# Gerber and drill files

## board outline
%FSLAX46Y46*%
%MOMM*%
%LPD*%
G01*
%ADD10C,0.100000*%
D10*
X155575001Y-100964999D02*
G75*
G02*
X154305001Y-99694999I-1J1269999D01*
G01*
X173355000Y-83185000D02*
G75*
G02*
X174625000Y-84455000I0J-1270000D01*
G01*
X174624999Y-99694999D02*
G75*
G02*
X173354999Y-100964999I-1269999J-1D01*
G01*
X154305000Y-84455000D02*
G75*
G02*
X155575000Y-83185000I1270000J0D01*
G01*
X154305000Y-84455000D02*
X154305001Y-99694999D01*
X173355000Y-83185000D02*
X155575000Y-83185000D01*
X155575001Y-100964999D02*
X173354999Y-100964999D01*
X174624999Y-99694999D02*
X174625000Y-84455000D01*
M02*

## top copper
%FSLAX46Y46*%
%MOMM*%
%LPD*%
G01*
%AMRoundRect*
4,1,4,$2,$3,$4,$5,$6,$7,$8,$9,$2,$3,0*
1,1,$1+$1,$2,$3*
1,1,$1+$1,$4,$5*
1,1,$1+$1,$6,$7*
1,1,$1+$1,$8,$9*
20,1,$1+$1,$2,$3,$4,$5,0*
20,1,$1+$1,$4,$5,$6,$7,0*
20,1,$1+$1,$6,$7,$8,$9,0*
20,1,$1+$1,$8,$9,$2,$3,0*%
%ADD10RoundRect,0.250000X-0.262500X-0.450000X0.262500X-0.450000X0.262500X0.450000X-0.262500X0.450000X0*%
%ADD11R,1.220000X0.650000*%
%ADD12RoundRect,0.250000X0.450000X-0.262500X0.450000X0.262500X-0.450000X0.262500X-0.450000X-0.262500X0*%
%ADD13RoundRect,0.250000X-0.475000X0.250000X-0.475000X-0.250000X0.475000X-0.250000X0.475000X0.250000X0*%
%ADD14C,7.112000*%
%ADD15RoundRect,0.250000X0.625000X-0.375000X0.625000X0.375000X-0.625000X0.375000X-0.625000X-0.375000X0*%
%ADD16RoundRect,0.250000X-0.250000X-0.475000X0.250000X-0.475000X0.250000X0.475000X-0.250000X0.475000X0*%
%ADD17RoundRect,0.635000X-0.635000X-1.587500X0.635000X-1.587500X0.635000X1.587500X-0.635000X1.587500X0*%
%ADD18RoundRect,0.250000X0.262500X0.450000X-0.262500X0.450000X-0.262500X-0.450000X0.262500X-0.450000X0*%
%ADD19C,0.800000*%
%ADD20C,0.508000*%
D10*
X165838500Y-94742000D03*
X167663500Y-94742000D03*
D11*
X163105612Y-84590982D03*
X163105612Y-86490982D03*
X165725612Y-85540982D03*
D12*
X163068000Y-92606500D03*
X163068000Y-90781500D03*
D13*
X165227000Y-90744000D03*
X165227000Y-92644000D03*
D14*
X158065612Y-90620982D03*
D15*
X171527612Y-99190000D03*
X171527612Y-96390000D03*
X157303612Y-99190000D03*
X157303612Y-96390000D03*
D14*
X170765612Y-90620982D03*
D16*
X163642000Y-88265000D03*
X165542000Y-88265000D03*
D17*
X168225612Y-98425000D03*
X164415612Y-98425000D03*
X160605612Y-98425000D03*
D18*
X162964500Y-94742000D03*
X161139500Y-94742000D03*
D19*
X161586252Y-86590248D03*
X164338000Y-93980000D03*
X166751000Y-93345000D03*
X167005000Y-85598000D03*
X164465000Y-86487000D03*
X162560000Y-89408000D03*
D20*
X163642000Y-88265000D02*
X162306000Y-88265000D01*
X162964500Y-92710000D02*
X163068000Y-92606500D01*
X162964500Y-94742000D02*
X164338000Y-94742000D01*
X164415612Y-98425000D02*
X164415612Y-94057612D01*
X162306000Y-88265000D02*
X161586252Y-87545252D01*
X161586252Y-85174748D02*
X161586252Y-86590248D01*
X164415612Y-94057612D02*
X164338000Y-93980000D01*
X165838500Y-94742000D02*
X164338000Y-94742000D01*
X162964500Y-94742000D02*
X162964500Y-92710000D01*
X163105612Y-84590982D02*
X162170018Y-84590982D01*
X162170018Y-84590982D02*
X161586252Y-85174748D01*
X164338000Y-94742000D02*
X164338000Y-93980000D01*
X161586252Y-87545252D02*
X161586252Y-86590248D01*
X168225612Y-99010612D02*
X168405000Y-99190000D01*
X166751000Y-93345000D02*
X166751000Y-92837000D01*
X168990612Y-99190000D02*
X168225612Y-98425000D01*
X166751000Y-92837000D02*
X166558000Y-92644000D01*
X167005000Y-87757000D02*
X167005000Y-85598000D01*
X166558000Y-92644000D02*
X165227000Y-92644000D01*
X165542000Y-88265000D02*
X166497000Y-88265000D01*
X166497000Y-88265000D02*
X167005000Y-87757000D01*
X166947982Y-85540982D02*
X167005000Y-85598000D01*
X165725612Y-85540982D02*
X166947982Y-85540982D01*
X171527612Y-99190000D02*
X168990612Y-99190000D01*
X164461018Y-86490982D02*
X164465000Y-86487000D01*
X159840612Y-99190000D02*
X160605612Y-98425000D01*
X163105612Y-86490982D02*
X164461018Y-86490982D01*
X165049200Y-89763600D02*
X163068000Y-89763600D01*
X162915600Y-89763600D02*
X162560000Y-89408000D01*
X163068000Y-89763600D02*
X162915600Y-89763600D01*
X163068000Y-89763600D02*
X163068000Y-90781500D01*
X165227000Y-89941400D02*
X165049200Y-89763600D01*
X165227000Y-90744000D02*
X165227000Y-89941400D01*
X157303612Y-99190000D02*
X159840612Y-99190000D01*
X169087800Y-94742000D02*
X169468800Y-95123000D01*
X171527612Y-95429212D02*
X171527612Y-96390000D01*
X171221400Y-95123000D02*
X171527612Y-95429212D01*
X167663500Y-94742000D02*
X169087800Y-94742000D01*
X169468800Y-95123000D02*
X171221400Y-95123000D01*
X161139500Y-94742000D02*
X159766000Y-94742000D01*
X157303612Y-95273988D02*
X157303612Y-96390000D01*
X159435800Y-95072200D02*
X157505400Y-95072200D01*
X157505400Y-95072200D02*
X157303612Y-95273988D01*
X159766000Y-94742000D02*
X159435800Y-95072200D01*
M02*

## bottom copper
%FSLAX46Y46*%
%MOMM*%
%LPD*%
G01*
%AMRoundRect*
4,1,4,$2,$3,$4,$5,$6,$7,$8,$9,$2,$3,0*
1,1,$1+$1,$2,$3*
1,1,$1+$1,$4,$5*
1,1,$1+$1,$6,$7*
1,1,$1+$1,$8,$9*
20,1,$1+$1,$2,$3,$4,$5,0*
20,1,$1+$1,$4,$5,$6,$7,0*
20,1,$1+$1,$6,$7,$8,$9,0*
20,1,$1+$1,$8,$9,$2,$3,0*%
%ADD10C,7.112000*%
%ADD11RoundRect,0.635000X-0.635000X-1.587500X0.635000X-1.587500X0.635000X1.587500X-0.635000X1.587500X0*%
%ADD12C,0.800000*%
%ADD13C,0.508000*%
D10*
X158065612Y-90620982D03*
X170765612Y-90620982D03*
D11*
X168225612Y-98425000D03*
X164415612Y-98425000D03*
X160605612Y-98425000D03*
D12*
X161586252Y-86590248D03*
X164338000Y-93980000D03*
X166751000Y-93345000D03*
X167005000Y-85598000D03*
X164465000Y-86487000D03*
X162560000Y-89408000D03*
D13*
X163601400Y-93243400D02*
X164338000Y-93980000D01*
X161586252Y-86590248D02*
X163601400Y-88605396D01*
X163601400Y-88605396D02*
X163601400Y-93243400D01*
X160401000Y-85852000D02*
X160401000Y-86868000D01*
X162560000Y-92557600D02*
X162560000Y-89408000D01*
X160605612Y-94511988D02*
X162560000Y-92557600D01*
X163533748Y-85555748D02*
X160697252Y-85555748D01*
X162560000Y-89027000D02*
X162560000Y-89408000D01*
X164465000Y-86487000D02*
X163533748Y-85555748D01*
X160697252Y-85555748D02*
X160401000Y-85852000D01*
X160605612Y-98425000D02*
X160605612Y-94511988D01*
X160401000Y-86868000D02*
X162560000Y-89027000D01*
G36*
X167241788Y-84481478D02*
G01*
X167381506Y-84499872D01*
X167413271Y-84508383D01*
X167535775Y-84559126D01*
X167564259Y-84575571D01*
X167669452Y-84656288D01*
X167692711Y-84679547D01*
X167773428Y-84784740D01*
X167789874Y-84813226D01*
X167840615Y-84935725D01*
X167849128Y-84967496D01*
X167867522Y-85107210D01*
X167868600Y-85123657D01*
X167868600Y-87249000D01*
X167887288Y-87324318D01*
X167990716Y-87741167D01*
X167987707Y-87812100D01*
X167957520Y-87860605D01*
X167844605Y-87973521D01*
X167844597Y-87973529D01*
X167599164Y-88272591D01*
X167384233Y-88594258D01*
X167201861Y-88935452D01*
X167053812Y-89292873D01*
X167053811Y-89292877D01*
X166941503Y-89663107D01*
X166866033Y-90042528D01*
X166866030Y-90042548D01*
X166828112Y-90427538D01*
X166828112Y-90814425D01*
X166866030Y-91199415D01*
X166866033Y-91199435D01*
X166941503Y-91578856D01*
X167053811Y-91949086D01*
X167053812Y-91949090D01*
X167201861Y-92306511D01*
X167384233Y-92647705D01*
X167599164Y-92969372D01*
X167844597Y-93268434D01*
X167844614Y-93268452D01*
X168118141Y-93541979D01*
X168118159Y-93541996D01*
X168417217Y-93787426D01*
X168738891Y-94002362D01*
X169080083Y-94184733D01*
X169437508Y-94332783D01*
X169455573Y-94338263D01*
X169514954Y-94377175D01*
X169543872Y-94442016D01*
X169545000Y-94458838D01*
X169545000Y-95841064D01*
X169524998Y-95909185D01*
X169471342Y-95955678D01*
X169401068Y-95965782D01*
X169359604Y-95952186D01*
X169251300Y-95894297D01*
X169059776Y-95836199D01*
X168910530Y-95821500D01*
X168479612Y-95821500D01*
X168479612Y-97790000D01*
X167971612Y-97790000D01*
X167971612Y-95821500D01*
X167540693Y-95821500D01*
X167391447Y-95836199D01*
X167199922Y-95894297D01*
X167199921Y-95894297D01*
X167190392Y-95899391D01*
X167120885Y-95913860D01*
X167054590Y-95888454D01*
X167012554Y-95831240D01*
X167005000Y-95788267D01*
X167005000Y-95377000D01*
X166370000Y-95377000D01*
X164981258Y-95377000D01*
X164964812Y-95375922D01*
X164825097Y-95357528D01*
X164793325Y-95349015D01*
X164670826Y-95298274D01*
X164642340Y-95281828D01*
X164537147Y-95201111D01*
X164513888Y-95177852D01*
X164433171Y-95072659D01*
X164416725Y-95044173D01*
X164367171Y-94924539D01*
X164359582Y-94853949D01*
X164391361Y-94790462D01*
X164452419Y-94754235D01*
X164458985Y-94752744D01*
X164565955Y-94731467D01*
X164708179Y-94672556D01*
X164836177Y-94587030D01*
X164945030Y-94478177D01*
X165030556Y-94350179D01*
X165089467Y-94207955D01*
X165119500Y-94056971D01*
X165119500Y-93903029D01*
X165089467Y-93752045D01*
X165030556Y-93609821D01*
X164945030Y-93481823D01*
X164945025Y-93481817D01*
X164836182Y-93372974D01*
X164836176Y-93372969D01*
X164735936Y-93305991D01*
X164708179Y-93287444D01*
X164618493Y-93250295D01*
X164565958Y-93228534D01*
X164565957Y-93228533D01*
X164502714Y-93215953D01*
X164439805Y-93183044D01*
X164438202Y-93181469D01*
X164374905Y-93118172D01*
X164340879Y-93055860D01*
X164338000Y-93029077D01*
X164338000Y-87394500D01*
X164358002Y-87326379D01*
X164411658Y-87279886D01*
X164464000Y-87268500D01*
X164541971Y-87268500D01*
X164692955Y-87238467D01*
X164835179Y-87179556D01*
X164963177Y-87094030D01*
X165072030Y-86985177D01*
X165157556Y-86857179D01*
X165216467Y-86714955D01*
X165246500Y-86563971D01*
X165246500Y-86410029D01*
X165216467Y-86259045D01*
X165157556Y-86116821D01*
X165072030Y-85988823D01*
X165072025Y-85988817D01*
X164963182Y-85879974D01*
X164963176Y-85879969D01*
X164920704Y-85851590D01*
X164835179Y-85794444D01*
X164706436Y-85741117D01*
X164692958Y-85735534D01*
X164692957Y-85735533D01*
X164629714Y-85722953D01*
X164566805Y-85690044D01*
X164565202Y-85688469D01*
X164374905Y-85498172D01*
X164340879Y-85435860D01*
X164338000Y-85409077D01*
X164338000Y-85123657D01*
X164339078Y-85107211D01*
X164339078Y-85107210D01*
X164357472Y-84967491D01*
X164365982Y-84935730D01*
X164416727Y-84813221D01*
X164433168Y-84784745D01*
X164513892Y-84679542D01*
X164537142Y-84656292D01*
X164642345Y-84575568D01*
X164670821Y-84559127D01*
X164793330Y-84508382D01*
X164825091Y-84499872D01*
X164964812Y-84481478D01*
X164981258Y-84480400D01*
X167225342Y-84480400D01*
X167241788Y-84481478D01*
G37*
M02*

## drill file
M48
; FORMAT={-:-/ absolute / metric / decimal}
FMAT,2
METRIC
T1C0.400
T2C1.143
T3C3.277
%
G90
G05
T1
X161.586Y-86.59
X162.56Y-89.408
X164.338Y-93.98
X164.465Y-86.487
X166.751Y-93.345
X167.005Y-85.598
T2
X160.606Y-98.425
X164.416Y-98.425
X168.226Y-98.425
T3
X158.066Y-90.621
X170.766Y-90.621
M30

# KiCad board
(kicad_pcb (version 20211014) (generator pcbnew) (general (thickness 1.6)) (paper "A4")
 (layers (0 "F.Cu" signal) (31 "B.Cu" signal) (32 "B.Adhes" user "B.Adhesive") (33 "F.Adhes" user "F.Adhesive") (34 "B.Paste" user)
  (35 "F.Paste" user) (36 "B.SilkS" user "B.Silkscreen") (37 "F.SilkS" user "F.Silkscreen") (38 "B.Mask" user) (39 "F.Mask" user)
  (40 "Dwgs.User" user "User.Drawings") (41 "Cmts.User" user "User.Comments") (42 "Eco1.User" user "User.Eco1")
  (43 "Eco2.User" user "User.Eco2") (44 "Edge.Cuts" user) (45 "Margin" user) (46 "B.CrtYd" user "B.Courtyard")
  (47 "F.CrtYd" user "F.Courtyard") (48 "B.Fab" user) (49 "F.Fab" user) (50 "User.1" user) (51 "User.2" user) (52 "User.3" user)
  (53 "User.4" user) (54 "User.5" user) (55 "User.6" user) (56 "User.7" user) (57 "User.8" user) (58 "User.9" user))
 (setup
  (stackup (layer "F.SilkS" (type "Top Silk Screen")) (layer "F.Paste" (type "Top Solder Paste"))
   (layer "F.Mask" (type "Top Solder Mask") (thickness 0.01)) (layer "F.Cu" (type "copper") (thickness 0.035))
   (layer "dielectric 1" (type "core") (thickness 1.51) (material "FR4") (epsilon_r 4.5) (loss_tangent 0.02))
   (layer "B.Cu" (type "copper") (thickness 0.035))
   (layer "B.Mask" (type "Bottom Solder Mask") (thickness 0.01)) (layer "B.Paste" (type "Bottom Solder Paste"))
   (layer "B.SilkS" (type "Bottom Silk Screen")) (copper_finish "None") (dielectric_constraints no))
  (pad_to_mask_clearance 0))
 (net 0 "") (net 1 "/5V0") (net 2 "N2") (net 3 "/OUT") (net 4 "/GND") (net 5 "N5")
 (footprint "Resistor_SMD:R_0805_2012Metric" (layer "F.Cu") (at 166.751 94.742)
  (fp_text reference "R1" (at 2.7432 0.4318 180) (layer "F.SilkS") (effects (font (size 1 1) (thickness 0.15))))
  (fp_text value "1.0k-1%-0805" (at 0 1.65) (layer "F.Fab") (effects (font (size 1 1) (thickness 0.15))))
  (pad "1" smd roundrect (at -0.9125 0) (size 1.025 1.4) (layers "F.Cu" "F.Paste" "F.Mask") (roundrect_rratio 0.243902) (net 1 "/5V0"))
  (pad "2" smd roundrect (at 0.9125 0) (size 1.025 1.4) (layers "F.Cu" "F.Paste" "F.Mask") (roundrect_rratio 0.243902) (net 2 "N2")))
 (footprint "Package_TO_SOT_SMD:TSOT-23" (layer "F.Cu") (at 164.415612 85.540982)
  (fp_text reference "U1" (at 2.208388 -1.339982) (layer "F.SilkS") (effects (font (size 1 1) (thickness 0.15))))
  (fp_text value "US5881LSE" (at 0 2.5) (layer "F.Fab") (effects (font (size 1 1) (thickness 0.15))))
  (pad "1" smd rect (at -1.31 -0.95) (size 1.22 0.65) (layers "F.Cu" "F.Paste" "F.Mask") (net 1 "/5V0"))
  (pad "2" smd rect (at -1.31 0.95) (size 1.22 0.65) (layers "F.Cu" "F.Paste" "F.Mask") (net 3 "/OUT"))
  (pad "3" smd rect (at 1.31 0) (size 1.22 0.65) (layers "F.Cu" "F.Paste" "F.Mask") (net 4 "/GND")))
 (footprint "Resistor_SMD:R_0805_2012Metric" (layer "F.Cu") (at 163.068 91.694 90)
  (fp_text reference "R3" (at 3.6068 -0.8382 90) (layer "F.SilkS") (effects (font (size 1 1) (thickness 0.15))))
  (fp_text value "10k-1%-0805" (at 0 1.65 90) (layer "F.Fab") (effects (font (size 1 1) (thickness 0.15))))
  (pad "1" smd roundrect (at -0.9125 0 90) (size 1.025 1.4) (layers "F.Cu" "F.Paste" "F.Mask") (roundrect_rratio 0.243902) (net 1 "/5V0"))
  (pad "2" smd roundrect (at 0.9125 0 90) (size 1.025 1.4) (layers "F.Cu" "F.Paste" "F.Mask") (roundrect_rratio 0.243902) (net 3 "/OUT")))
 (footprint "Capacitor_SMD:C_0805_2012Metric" (layer "F.Cu") (at 165.227 91.694 -90)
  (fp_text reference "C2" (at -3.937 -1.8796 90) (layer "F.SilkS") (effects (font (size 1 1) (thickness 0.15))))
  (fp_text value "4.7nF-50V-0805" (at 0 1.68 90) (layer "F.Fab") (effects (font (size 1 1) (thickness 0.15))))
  (pad "1" smd roundrect (at -0.95 0 270) (size 1 1.45) (layers "F.Cu" "F.Paste" "F.Mask") (roundrect_rratio 0.25) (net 3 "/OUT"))
  (pad "2" smd roundrect (at 0.95 0 270) (size 1 1.45) (layers "F.Cu" "F.Paste" "F.Mask") (roundrect_rratio 0.25) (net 4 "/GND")))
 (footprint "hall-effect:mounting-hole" (layer "F.Cu") (at 158.065612 90.620982)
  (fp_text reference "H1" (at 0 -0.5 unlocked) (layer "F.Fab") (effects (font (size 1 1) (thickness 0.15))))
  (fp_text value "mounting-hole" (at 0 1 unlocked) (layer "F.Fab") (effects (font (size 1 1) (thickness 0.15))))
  (pad "" np_thru_hole circle (at 0 0 90) (size 7.112 7.112) (drill 3.2766) (layers F&B.Cu *.Mask)))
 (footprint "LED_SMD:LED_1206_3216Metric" (layer "F.Cu") (at 171.527612 97.79 90)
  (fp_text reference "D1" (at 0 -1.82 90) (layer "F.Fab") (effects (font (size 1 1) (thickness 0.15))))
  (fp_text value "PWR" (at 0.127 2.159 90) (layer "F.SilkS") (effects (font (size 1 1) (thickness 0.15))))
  (pad "1" smd roundrect (at -1.4 0 90) (size 1.25 1.75) (layers "F.Cu" "F.Paste" "F.Mask") (roundrect_rratio 0.2) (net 4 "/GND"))
  (pad "2" smd roundrect (at 1.4 0 90) (size 1.25 1.75) (layers "F.Cu" "F.Paste" "F.Mask") (roundrect_rratio 0.2) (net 2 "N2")))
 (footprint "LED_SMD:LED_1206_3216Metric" (layer "F.Cu") (at 157.303612 97.79 90)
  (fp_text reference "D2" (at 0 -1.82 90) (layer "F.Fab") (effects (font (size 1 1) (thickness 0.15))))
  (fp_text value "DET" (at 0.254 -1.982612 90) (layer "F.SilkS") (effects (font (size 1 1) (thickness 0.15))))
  (pad "1" smd roundrect (at -1.4 0 90) (size 1.25 1.75) (layers "F.Cu" "F.Paste" "F.Mask") (roundrect_rratio 0.2) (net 3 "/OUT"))
  (pad "2" smd roundrect (at 1.4 0 90) (size 1.25 1.75) (layers "F.Cu" "F.Paste" "F.Mask") (roundrect_rratio 0.2) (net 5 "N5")))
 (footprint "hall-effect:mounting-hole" (layer "F.Cu") (at 170.765612 90.620982)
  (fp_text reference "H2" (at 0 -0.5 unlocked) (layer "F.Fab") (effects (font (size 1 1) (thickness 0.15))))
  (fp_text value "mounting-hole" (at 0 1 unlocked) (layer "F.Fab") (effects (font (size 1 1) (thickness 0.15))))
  (pad "" np_thru_hole circle (at 0 0 90) (size 7.112 7.112) (drill 3.2766) (layers F&B.Cu *.Mask)))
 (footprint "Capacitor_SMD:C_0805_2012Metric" (layer "F.Cu") (at 164.592 88.265)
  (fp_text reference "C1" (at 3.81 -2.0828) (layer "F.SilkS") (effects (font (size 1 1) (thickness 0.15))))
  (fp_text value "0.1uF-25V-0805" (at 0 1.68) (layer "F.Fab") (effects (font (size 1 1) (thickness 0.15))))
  (pad "1" smd roundrect (at -0.95 0) (size 1 1.45) (layers "F.Cu" "F.Paste" "F.Mask") (roundrect_rratio 0.25) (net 1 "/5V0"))
  (pad "2" smd roundrect (at 0.95 0) (size 1 1.45) (layers "F.Cu" "F.Paste" "F.Mask") (roundrect_rratio 0.25) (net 4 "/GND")))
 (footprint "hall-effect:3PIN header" (layer "F.Cu") (at 160.605612 98.425)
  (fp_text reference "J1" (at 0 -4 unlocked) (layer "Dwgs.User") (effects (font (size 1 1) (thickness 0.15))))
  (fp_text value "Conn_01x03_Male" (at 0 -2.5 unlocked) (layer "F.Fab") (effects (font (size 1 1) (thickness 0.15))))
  (pad "1" thru_hole roundrect (at 7.62 0) (size 2.54 4.445) (drill 1.143) (layers *.Cu *.Mask) (roundrect_rratio 0.25) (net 4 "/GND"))
  (pad "2" thru_hole roundrect locked (at 3.81 0) (size 2.54 4.445) (drill 1.143) (layers *.Cu *.Mask) (roundrect_rratio 0.25)
   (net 1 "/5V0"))
  (pad "3" thru_hole roundrect locked (at 0 0) (size 2.54 4.445) (drill 1.143) (layers *.Cu *.Mask) (roundrect_rratio 0.25) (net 3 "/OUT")))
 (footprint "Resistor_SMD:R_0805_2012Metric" (layer "F.Cu") (at 162.052 94.742 180)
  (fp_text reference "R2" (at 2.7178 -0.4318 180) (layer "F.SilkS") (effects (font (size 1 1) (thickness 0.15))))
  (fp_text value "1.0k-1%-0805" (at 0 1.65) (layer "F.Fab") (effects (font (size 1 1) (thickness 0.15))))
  (pad "1" smd roundrect (at -0.9125 0 180) (size 1.025 1.4) (layers "F.Cu" "F.Paste" "F.Mask") (roundrect_rratio 0.243902) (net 1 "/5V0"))
  (pad "2" smd roundrect (at 0.9125 0 180) (size 1.025 1.4) (layers "F.Cu" "F.Paste" "F.Mask") (roundrect_rratio 0.243902) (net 5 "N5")))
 (gr_arc (start 155.575001 100.964999) (mid 154.676975 100.593025) (end 154.305001 99.694999) (layer "Edge.Cuts") (width 0.1))
 (gr_arc (start 173.355 83.185) (mid 174.253026 83.556974) (end 174.625 84.455) (layer "Edge.Cuts") (width 0.1))
 (gr_arc (start 174.624999 99.694999) (mid 174.253025 100.593025) (end 173.354999 100.964999) (layer "Edge.Cuts") (width 0.1))
 (gr_arc (start 154.305 84.455) (mid 154.676974 83.556974) (end 155.575 83.185) (layer "Edge.Cuts") (width 0.1))
 (gr_line (start 154.305 84.455) (end 154.305001 99.694999) (layer "Edge.Cuts") (width 0.1))
 (gr_line (start 173.355 83.185) (end 155.575 83.185) (layer "Edge.Cuts") (width 0.1))
 (gr_line (start 155.575001 100.964999) (end 173.354999 100.964999) (layer "Edge.Cuts") (width 0.1))
 (gr_line (start 174.624999 99.694999) (end 174.625 84.455) (layer "Edge.Cuts") (width 0.1))
 (segment (start 163.642 88.265) (end 162.306 88.265) (width 0.508) (layer "F.Cu") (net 1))
 (segment (start 162.9645 92.71) (end 163.068 92.6065) (width 0.508) (layer "F.Cu") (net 1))
 (segment (start 162.9645 94.742) (end 164.338 94.742) (width 0.508) (layer "F.Cu") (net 1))
 (segment (start 164.415612 98.425) (end 164.415612 94.057612) (width 0.508) (layer "F.Cu") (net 1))
 (segment (start 162.306 88.265) (end 161.586252 87.545252) (width 0.508) (layer "F.Cu") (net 1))
 (segment (start 161.586252 85.174748) (end 161.586252 86.590248) (width 0.508) (layer "F.Cu") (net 1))
 (segment (start 164.415612 94.057612) (end 164.338 93.98) (width 0.508) (layer "F.Cu") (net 1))
 (segment (start 165.8385 94.742) (end 164.338 94.742) (width 0.508) (layer "F.Cu") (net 1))
 (segment (start 162.9645 94.742) (end 162.9645 92.71) (width 0.508) (layer "F.Cu") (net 1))
 (segment (start 163.105612 84.590982) (end 162.170018 84.590982) (width 0.508) (layer "F.Cu") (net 1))
 (segment (start 162.170018 84.590982) (end 161.586252 85.174748) (width 0.508) (layer "F.Cu") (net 1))
 (segment (start 164.338 94.742) (end 164.338 93.98) (width 0.508) (layer "F.Cu") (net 1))
 (segment (start 161.586252 87.545252) (end 161.586252 86.590248) (width 0.508) (layer "F.Cu") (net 1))
 (via (at 161.586252 86.590248) (size 0.8) (drill 0.4) (layers "F.Cu" "B.Cu") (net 1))
 (via (at 164.338 93.98) (size 0.8) (drill 0.4) (layers "F.Cu" "B.Cu") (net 1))
 (segment (start 163.6014 93.2434) (end 164.338 93.98) (width 0.508) (layer "B.Cu") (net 1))
 (segment (start 161.586252 86.590248) (end 163.6014 88.605396) (width 0.508) (layer "B.Cu") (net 1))
 (segment (start 163.6014 88.605396) (end 163.6014 93.2434) (width 0.508) (layer "B.Cu") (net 1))
 (segment (start 168.225612 99.010612) (end 168.405 99.19) (width 0.508) (layer "F.Cu") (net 4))
 (segment (start 166.751 93.345) (end 166.751 92.837) (width 0.508) (layer "F.Cu") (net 4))
 (segment (start 168.990612 99.19) (end 168.225612 98.425) (width 0.508) (layer "F.Cu") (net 4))
 (segment (start 166.751 92.837) (end 166.558 92.644) (width 0.508) (layer "F.Cu") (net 4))
 (segment (start 167.005 87.757) (end 167.005 85.598) (width 0.508) (layer "F.Cu") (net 4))
 (segment (start 166.558 92.644) (end 165.227 92.644) (width 0.508) (layer "F.Cu") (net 4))
 (segment (start 165.542 88.265) (end 166.497 88.265) (width 0.508) (layer "F.Cu") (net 4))
 (segment (start 166.497 88.265) (end 167.005 87.757) (width 0.508) (layer "F.Cu") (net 4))
 (segment (start 166.947982 85.540982) (end 167.005 85.598) (width 0.508) (layer "F.Cu") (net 4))
 (segment (start 165.725612 85.540982) (end 166.947982 85.540982) (width 0.508) (layer "F.Cu") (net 4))
 (segment (start 171.527612 99.19) (end 168.990612 99.19) (width 0.508) (layer "F.Cu") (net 4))
 (via (at 166.751 93.345) (size 0.8) (drill 0.4) (layers "F.Cu" "B.Cu") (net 4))
 (via (at 167.005 85.598) (size 0.8) (drill 0.4) (layers "F.Cu" "B.Cu") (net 4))
 (segment (start 164.461018 86.490982) (end 164.465 86.487) (width 0.508) (layer "F.Cu") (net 3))
 (segment (start 159.840612 99.19) (end 160.605612 98.425) (width 0.508) (layer "F.Cu") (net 3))
 (segment (start 163.105612 86.490982) (end 164.461018 86.490982) (width 0.508) (layer "F.Cu") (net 3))
 (segment (start 165.0492 89.7636) (end 163.068 89.7636) (width 0.508) (layer "F.Cu") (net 3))
 (segment (start 162.9156 89.7636) (end 162.56 89.408) (width 0.508) (layer "F.Cu") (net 3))
 (segment (start 163.068 89.7636) (end 162.9156 89.7636) (width 0.508) (layer "F.Cu") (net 3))
 (segment (start 163.068 89.7636) (end 163.068 90.7815) (width 0.508) (layer "F.Cu") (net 3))
 (segment (start 165.227 89.9414) (end 165.0492 89.7636) (width 0.508) (layer "F.Cu") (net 3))
 (segment (start 165.227 90.744) (end 165.227 89.9414) (width 0.508) (layer "F.Cu") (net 3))
 (segment (start 157.303612 99.19) (end 159.840612 99.19) (width 0.508) (layer "F.Cu") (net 3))
 (via (at 164.465 86.487) (size 0.8) (drill 0.4) (layers "F.Cu" "B.Cu") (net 3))
 (via (at 162.56 89.408) (size 0.8) (drill 0.4) (layers "F.Cu" "B.Cu") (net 3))
 (segment (start 160.401 85.852) (end 160.401 86.868) (width 0.508) (layer "B.Cu") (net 3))
 (segment (start 162.56 92.5576) (end 162.56 89.408) (width 0.508) (layer "B.Cu") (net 3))
 (segment (start 160.605612 94.511988) (end 162.56 92.5576) (width 0.508) (layer "B.Cu") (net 3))
 (segment (start 163.533748 85.555748) (end 160.697252 85.555748) (width 0.508) (layer "B.Cu") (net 3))
 (segment (start 162.56 89.027) (end 162.56 89.408) (width 0.508) (layer "B.Cu") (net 3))
 (segment (start 164.465 86.487) (end 163.533748 85.555748) (width 0.508) (layer "B.Cu") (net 3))
 (segment (start 160.697252 85.555748) (end 160.401 85.852) (width 0.508) (layer "B.Cu") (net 3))
 (segment (start 160.605612 98.425) (end 160.605612 94.511988) (width 0.508) (layer "B.Cu") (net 3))
 (segment (start 160.401 86.868) (end 162.56 89.027) (width 0.508) (layer "B.Cu") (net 3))
 (segment (start 169.0878 94.742) (end 169.4688 95.123) (width 0.508) (layer "F.Cu") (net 2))
 (segment (start 171.527612 95.429212) (end 171.527612 96.39) (width 0.508) (layer "F.Cu") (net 2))
 (segment (start 171.2214 95.123) (end 171.527612 95.429212) (width 0.508) (layer "F.Cu") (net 2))
 (segment (start 167.6635 94.742) (end 169.0878 94.742) (width 0.508) (layer "F.Cu") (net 2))
 (segment (start 169.4688 95.123) (end 171.2214 95.123) (width 0.508) (layer "F.Cu") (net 2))
 (segment (start 161.1395 94.742) (end 159.766 94.742) (width 0.508) (layer "F.Cu") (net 5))
 (segment (start 157.303612 95.273988) (end 157.303612 96.39) (width 0.508) (layer "F.Cu") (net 5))
 (segment (start 159.4358 95.0722) (end 157.5054 95.0722) (width 0.508) (layer "F.Cu") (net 5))
 (segment (start 157.5054 95.0722) (end 157.303612 95.273988) (width 0.508) (layer "F.Cu") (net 5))
 (segment (start 159.766 94.742) (end 159.4358 95.0722) (width 0.508) (layer "F.Cu") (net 5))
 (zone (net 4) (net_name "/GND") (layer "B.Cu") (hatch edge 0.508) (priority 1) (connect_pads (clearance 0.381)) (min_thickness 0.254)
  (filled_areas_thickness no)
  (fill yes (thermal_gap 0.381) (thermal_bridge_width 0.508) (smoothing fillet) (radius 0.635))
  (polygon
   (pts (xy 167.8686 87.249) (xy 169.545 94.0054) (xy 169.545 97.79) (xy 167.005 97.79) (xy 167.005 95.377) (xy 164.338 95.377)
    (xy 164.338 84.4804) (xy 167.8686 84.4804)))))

